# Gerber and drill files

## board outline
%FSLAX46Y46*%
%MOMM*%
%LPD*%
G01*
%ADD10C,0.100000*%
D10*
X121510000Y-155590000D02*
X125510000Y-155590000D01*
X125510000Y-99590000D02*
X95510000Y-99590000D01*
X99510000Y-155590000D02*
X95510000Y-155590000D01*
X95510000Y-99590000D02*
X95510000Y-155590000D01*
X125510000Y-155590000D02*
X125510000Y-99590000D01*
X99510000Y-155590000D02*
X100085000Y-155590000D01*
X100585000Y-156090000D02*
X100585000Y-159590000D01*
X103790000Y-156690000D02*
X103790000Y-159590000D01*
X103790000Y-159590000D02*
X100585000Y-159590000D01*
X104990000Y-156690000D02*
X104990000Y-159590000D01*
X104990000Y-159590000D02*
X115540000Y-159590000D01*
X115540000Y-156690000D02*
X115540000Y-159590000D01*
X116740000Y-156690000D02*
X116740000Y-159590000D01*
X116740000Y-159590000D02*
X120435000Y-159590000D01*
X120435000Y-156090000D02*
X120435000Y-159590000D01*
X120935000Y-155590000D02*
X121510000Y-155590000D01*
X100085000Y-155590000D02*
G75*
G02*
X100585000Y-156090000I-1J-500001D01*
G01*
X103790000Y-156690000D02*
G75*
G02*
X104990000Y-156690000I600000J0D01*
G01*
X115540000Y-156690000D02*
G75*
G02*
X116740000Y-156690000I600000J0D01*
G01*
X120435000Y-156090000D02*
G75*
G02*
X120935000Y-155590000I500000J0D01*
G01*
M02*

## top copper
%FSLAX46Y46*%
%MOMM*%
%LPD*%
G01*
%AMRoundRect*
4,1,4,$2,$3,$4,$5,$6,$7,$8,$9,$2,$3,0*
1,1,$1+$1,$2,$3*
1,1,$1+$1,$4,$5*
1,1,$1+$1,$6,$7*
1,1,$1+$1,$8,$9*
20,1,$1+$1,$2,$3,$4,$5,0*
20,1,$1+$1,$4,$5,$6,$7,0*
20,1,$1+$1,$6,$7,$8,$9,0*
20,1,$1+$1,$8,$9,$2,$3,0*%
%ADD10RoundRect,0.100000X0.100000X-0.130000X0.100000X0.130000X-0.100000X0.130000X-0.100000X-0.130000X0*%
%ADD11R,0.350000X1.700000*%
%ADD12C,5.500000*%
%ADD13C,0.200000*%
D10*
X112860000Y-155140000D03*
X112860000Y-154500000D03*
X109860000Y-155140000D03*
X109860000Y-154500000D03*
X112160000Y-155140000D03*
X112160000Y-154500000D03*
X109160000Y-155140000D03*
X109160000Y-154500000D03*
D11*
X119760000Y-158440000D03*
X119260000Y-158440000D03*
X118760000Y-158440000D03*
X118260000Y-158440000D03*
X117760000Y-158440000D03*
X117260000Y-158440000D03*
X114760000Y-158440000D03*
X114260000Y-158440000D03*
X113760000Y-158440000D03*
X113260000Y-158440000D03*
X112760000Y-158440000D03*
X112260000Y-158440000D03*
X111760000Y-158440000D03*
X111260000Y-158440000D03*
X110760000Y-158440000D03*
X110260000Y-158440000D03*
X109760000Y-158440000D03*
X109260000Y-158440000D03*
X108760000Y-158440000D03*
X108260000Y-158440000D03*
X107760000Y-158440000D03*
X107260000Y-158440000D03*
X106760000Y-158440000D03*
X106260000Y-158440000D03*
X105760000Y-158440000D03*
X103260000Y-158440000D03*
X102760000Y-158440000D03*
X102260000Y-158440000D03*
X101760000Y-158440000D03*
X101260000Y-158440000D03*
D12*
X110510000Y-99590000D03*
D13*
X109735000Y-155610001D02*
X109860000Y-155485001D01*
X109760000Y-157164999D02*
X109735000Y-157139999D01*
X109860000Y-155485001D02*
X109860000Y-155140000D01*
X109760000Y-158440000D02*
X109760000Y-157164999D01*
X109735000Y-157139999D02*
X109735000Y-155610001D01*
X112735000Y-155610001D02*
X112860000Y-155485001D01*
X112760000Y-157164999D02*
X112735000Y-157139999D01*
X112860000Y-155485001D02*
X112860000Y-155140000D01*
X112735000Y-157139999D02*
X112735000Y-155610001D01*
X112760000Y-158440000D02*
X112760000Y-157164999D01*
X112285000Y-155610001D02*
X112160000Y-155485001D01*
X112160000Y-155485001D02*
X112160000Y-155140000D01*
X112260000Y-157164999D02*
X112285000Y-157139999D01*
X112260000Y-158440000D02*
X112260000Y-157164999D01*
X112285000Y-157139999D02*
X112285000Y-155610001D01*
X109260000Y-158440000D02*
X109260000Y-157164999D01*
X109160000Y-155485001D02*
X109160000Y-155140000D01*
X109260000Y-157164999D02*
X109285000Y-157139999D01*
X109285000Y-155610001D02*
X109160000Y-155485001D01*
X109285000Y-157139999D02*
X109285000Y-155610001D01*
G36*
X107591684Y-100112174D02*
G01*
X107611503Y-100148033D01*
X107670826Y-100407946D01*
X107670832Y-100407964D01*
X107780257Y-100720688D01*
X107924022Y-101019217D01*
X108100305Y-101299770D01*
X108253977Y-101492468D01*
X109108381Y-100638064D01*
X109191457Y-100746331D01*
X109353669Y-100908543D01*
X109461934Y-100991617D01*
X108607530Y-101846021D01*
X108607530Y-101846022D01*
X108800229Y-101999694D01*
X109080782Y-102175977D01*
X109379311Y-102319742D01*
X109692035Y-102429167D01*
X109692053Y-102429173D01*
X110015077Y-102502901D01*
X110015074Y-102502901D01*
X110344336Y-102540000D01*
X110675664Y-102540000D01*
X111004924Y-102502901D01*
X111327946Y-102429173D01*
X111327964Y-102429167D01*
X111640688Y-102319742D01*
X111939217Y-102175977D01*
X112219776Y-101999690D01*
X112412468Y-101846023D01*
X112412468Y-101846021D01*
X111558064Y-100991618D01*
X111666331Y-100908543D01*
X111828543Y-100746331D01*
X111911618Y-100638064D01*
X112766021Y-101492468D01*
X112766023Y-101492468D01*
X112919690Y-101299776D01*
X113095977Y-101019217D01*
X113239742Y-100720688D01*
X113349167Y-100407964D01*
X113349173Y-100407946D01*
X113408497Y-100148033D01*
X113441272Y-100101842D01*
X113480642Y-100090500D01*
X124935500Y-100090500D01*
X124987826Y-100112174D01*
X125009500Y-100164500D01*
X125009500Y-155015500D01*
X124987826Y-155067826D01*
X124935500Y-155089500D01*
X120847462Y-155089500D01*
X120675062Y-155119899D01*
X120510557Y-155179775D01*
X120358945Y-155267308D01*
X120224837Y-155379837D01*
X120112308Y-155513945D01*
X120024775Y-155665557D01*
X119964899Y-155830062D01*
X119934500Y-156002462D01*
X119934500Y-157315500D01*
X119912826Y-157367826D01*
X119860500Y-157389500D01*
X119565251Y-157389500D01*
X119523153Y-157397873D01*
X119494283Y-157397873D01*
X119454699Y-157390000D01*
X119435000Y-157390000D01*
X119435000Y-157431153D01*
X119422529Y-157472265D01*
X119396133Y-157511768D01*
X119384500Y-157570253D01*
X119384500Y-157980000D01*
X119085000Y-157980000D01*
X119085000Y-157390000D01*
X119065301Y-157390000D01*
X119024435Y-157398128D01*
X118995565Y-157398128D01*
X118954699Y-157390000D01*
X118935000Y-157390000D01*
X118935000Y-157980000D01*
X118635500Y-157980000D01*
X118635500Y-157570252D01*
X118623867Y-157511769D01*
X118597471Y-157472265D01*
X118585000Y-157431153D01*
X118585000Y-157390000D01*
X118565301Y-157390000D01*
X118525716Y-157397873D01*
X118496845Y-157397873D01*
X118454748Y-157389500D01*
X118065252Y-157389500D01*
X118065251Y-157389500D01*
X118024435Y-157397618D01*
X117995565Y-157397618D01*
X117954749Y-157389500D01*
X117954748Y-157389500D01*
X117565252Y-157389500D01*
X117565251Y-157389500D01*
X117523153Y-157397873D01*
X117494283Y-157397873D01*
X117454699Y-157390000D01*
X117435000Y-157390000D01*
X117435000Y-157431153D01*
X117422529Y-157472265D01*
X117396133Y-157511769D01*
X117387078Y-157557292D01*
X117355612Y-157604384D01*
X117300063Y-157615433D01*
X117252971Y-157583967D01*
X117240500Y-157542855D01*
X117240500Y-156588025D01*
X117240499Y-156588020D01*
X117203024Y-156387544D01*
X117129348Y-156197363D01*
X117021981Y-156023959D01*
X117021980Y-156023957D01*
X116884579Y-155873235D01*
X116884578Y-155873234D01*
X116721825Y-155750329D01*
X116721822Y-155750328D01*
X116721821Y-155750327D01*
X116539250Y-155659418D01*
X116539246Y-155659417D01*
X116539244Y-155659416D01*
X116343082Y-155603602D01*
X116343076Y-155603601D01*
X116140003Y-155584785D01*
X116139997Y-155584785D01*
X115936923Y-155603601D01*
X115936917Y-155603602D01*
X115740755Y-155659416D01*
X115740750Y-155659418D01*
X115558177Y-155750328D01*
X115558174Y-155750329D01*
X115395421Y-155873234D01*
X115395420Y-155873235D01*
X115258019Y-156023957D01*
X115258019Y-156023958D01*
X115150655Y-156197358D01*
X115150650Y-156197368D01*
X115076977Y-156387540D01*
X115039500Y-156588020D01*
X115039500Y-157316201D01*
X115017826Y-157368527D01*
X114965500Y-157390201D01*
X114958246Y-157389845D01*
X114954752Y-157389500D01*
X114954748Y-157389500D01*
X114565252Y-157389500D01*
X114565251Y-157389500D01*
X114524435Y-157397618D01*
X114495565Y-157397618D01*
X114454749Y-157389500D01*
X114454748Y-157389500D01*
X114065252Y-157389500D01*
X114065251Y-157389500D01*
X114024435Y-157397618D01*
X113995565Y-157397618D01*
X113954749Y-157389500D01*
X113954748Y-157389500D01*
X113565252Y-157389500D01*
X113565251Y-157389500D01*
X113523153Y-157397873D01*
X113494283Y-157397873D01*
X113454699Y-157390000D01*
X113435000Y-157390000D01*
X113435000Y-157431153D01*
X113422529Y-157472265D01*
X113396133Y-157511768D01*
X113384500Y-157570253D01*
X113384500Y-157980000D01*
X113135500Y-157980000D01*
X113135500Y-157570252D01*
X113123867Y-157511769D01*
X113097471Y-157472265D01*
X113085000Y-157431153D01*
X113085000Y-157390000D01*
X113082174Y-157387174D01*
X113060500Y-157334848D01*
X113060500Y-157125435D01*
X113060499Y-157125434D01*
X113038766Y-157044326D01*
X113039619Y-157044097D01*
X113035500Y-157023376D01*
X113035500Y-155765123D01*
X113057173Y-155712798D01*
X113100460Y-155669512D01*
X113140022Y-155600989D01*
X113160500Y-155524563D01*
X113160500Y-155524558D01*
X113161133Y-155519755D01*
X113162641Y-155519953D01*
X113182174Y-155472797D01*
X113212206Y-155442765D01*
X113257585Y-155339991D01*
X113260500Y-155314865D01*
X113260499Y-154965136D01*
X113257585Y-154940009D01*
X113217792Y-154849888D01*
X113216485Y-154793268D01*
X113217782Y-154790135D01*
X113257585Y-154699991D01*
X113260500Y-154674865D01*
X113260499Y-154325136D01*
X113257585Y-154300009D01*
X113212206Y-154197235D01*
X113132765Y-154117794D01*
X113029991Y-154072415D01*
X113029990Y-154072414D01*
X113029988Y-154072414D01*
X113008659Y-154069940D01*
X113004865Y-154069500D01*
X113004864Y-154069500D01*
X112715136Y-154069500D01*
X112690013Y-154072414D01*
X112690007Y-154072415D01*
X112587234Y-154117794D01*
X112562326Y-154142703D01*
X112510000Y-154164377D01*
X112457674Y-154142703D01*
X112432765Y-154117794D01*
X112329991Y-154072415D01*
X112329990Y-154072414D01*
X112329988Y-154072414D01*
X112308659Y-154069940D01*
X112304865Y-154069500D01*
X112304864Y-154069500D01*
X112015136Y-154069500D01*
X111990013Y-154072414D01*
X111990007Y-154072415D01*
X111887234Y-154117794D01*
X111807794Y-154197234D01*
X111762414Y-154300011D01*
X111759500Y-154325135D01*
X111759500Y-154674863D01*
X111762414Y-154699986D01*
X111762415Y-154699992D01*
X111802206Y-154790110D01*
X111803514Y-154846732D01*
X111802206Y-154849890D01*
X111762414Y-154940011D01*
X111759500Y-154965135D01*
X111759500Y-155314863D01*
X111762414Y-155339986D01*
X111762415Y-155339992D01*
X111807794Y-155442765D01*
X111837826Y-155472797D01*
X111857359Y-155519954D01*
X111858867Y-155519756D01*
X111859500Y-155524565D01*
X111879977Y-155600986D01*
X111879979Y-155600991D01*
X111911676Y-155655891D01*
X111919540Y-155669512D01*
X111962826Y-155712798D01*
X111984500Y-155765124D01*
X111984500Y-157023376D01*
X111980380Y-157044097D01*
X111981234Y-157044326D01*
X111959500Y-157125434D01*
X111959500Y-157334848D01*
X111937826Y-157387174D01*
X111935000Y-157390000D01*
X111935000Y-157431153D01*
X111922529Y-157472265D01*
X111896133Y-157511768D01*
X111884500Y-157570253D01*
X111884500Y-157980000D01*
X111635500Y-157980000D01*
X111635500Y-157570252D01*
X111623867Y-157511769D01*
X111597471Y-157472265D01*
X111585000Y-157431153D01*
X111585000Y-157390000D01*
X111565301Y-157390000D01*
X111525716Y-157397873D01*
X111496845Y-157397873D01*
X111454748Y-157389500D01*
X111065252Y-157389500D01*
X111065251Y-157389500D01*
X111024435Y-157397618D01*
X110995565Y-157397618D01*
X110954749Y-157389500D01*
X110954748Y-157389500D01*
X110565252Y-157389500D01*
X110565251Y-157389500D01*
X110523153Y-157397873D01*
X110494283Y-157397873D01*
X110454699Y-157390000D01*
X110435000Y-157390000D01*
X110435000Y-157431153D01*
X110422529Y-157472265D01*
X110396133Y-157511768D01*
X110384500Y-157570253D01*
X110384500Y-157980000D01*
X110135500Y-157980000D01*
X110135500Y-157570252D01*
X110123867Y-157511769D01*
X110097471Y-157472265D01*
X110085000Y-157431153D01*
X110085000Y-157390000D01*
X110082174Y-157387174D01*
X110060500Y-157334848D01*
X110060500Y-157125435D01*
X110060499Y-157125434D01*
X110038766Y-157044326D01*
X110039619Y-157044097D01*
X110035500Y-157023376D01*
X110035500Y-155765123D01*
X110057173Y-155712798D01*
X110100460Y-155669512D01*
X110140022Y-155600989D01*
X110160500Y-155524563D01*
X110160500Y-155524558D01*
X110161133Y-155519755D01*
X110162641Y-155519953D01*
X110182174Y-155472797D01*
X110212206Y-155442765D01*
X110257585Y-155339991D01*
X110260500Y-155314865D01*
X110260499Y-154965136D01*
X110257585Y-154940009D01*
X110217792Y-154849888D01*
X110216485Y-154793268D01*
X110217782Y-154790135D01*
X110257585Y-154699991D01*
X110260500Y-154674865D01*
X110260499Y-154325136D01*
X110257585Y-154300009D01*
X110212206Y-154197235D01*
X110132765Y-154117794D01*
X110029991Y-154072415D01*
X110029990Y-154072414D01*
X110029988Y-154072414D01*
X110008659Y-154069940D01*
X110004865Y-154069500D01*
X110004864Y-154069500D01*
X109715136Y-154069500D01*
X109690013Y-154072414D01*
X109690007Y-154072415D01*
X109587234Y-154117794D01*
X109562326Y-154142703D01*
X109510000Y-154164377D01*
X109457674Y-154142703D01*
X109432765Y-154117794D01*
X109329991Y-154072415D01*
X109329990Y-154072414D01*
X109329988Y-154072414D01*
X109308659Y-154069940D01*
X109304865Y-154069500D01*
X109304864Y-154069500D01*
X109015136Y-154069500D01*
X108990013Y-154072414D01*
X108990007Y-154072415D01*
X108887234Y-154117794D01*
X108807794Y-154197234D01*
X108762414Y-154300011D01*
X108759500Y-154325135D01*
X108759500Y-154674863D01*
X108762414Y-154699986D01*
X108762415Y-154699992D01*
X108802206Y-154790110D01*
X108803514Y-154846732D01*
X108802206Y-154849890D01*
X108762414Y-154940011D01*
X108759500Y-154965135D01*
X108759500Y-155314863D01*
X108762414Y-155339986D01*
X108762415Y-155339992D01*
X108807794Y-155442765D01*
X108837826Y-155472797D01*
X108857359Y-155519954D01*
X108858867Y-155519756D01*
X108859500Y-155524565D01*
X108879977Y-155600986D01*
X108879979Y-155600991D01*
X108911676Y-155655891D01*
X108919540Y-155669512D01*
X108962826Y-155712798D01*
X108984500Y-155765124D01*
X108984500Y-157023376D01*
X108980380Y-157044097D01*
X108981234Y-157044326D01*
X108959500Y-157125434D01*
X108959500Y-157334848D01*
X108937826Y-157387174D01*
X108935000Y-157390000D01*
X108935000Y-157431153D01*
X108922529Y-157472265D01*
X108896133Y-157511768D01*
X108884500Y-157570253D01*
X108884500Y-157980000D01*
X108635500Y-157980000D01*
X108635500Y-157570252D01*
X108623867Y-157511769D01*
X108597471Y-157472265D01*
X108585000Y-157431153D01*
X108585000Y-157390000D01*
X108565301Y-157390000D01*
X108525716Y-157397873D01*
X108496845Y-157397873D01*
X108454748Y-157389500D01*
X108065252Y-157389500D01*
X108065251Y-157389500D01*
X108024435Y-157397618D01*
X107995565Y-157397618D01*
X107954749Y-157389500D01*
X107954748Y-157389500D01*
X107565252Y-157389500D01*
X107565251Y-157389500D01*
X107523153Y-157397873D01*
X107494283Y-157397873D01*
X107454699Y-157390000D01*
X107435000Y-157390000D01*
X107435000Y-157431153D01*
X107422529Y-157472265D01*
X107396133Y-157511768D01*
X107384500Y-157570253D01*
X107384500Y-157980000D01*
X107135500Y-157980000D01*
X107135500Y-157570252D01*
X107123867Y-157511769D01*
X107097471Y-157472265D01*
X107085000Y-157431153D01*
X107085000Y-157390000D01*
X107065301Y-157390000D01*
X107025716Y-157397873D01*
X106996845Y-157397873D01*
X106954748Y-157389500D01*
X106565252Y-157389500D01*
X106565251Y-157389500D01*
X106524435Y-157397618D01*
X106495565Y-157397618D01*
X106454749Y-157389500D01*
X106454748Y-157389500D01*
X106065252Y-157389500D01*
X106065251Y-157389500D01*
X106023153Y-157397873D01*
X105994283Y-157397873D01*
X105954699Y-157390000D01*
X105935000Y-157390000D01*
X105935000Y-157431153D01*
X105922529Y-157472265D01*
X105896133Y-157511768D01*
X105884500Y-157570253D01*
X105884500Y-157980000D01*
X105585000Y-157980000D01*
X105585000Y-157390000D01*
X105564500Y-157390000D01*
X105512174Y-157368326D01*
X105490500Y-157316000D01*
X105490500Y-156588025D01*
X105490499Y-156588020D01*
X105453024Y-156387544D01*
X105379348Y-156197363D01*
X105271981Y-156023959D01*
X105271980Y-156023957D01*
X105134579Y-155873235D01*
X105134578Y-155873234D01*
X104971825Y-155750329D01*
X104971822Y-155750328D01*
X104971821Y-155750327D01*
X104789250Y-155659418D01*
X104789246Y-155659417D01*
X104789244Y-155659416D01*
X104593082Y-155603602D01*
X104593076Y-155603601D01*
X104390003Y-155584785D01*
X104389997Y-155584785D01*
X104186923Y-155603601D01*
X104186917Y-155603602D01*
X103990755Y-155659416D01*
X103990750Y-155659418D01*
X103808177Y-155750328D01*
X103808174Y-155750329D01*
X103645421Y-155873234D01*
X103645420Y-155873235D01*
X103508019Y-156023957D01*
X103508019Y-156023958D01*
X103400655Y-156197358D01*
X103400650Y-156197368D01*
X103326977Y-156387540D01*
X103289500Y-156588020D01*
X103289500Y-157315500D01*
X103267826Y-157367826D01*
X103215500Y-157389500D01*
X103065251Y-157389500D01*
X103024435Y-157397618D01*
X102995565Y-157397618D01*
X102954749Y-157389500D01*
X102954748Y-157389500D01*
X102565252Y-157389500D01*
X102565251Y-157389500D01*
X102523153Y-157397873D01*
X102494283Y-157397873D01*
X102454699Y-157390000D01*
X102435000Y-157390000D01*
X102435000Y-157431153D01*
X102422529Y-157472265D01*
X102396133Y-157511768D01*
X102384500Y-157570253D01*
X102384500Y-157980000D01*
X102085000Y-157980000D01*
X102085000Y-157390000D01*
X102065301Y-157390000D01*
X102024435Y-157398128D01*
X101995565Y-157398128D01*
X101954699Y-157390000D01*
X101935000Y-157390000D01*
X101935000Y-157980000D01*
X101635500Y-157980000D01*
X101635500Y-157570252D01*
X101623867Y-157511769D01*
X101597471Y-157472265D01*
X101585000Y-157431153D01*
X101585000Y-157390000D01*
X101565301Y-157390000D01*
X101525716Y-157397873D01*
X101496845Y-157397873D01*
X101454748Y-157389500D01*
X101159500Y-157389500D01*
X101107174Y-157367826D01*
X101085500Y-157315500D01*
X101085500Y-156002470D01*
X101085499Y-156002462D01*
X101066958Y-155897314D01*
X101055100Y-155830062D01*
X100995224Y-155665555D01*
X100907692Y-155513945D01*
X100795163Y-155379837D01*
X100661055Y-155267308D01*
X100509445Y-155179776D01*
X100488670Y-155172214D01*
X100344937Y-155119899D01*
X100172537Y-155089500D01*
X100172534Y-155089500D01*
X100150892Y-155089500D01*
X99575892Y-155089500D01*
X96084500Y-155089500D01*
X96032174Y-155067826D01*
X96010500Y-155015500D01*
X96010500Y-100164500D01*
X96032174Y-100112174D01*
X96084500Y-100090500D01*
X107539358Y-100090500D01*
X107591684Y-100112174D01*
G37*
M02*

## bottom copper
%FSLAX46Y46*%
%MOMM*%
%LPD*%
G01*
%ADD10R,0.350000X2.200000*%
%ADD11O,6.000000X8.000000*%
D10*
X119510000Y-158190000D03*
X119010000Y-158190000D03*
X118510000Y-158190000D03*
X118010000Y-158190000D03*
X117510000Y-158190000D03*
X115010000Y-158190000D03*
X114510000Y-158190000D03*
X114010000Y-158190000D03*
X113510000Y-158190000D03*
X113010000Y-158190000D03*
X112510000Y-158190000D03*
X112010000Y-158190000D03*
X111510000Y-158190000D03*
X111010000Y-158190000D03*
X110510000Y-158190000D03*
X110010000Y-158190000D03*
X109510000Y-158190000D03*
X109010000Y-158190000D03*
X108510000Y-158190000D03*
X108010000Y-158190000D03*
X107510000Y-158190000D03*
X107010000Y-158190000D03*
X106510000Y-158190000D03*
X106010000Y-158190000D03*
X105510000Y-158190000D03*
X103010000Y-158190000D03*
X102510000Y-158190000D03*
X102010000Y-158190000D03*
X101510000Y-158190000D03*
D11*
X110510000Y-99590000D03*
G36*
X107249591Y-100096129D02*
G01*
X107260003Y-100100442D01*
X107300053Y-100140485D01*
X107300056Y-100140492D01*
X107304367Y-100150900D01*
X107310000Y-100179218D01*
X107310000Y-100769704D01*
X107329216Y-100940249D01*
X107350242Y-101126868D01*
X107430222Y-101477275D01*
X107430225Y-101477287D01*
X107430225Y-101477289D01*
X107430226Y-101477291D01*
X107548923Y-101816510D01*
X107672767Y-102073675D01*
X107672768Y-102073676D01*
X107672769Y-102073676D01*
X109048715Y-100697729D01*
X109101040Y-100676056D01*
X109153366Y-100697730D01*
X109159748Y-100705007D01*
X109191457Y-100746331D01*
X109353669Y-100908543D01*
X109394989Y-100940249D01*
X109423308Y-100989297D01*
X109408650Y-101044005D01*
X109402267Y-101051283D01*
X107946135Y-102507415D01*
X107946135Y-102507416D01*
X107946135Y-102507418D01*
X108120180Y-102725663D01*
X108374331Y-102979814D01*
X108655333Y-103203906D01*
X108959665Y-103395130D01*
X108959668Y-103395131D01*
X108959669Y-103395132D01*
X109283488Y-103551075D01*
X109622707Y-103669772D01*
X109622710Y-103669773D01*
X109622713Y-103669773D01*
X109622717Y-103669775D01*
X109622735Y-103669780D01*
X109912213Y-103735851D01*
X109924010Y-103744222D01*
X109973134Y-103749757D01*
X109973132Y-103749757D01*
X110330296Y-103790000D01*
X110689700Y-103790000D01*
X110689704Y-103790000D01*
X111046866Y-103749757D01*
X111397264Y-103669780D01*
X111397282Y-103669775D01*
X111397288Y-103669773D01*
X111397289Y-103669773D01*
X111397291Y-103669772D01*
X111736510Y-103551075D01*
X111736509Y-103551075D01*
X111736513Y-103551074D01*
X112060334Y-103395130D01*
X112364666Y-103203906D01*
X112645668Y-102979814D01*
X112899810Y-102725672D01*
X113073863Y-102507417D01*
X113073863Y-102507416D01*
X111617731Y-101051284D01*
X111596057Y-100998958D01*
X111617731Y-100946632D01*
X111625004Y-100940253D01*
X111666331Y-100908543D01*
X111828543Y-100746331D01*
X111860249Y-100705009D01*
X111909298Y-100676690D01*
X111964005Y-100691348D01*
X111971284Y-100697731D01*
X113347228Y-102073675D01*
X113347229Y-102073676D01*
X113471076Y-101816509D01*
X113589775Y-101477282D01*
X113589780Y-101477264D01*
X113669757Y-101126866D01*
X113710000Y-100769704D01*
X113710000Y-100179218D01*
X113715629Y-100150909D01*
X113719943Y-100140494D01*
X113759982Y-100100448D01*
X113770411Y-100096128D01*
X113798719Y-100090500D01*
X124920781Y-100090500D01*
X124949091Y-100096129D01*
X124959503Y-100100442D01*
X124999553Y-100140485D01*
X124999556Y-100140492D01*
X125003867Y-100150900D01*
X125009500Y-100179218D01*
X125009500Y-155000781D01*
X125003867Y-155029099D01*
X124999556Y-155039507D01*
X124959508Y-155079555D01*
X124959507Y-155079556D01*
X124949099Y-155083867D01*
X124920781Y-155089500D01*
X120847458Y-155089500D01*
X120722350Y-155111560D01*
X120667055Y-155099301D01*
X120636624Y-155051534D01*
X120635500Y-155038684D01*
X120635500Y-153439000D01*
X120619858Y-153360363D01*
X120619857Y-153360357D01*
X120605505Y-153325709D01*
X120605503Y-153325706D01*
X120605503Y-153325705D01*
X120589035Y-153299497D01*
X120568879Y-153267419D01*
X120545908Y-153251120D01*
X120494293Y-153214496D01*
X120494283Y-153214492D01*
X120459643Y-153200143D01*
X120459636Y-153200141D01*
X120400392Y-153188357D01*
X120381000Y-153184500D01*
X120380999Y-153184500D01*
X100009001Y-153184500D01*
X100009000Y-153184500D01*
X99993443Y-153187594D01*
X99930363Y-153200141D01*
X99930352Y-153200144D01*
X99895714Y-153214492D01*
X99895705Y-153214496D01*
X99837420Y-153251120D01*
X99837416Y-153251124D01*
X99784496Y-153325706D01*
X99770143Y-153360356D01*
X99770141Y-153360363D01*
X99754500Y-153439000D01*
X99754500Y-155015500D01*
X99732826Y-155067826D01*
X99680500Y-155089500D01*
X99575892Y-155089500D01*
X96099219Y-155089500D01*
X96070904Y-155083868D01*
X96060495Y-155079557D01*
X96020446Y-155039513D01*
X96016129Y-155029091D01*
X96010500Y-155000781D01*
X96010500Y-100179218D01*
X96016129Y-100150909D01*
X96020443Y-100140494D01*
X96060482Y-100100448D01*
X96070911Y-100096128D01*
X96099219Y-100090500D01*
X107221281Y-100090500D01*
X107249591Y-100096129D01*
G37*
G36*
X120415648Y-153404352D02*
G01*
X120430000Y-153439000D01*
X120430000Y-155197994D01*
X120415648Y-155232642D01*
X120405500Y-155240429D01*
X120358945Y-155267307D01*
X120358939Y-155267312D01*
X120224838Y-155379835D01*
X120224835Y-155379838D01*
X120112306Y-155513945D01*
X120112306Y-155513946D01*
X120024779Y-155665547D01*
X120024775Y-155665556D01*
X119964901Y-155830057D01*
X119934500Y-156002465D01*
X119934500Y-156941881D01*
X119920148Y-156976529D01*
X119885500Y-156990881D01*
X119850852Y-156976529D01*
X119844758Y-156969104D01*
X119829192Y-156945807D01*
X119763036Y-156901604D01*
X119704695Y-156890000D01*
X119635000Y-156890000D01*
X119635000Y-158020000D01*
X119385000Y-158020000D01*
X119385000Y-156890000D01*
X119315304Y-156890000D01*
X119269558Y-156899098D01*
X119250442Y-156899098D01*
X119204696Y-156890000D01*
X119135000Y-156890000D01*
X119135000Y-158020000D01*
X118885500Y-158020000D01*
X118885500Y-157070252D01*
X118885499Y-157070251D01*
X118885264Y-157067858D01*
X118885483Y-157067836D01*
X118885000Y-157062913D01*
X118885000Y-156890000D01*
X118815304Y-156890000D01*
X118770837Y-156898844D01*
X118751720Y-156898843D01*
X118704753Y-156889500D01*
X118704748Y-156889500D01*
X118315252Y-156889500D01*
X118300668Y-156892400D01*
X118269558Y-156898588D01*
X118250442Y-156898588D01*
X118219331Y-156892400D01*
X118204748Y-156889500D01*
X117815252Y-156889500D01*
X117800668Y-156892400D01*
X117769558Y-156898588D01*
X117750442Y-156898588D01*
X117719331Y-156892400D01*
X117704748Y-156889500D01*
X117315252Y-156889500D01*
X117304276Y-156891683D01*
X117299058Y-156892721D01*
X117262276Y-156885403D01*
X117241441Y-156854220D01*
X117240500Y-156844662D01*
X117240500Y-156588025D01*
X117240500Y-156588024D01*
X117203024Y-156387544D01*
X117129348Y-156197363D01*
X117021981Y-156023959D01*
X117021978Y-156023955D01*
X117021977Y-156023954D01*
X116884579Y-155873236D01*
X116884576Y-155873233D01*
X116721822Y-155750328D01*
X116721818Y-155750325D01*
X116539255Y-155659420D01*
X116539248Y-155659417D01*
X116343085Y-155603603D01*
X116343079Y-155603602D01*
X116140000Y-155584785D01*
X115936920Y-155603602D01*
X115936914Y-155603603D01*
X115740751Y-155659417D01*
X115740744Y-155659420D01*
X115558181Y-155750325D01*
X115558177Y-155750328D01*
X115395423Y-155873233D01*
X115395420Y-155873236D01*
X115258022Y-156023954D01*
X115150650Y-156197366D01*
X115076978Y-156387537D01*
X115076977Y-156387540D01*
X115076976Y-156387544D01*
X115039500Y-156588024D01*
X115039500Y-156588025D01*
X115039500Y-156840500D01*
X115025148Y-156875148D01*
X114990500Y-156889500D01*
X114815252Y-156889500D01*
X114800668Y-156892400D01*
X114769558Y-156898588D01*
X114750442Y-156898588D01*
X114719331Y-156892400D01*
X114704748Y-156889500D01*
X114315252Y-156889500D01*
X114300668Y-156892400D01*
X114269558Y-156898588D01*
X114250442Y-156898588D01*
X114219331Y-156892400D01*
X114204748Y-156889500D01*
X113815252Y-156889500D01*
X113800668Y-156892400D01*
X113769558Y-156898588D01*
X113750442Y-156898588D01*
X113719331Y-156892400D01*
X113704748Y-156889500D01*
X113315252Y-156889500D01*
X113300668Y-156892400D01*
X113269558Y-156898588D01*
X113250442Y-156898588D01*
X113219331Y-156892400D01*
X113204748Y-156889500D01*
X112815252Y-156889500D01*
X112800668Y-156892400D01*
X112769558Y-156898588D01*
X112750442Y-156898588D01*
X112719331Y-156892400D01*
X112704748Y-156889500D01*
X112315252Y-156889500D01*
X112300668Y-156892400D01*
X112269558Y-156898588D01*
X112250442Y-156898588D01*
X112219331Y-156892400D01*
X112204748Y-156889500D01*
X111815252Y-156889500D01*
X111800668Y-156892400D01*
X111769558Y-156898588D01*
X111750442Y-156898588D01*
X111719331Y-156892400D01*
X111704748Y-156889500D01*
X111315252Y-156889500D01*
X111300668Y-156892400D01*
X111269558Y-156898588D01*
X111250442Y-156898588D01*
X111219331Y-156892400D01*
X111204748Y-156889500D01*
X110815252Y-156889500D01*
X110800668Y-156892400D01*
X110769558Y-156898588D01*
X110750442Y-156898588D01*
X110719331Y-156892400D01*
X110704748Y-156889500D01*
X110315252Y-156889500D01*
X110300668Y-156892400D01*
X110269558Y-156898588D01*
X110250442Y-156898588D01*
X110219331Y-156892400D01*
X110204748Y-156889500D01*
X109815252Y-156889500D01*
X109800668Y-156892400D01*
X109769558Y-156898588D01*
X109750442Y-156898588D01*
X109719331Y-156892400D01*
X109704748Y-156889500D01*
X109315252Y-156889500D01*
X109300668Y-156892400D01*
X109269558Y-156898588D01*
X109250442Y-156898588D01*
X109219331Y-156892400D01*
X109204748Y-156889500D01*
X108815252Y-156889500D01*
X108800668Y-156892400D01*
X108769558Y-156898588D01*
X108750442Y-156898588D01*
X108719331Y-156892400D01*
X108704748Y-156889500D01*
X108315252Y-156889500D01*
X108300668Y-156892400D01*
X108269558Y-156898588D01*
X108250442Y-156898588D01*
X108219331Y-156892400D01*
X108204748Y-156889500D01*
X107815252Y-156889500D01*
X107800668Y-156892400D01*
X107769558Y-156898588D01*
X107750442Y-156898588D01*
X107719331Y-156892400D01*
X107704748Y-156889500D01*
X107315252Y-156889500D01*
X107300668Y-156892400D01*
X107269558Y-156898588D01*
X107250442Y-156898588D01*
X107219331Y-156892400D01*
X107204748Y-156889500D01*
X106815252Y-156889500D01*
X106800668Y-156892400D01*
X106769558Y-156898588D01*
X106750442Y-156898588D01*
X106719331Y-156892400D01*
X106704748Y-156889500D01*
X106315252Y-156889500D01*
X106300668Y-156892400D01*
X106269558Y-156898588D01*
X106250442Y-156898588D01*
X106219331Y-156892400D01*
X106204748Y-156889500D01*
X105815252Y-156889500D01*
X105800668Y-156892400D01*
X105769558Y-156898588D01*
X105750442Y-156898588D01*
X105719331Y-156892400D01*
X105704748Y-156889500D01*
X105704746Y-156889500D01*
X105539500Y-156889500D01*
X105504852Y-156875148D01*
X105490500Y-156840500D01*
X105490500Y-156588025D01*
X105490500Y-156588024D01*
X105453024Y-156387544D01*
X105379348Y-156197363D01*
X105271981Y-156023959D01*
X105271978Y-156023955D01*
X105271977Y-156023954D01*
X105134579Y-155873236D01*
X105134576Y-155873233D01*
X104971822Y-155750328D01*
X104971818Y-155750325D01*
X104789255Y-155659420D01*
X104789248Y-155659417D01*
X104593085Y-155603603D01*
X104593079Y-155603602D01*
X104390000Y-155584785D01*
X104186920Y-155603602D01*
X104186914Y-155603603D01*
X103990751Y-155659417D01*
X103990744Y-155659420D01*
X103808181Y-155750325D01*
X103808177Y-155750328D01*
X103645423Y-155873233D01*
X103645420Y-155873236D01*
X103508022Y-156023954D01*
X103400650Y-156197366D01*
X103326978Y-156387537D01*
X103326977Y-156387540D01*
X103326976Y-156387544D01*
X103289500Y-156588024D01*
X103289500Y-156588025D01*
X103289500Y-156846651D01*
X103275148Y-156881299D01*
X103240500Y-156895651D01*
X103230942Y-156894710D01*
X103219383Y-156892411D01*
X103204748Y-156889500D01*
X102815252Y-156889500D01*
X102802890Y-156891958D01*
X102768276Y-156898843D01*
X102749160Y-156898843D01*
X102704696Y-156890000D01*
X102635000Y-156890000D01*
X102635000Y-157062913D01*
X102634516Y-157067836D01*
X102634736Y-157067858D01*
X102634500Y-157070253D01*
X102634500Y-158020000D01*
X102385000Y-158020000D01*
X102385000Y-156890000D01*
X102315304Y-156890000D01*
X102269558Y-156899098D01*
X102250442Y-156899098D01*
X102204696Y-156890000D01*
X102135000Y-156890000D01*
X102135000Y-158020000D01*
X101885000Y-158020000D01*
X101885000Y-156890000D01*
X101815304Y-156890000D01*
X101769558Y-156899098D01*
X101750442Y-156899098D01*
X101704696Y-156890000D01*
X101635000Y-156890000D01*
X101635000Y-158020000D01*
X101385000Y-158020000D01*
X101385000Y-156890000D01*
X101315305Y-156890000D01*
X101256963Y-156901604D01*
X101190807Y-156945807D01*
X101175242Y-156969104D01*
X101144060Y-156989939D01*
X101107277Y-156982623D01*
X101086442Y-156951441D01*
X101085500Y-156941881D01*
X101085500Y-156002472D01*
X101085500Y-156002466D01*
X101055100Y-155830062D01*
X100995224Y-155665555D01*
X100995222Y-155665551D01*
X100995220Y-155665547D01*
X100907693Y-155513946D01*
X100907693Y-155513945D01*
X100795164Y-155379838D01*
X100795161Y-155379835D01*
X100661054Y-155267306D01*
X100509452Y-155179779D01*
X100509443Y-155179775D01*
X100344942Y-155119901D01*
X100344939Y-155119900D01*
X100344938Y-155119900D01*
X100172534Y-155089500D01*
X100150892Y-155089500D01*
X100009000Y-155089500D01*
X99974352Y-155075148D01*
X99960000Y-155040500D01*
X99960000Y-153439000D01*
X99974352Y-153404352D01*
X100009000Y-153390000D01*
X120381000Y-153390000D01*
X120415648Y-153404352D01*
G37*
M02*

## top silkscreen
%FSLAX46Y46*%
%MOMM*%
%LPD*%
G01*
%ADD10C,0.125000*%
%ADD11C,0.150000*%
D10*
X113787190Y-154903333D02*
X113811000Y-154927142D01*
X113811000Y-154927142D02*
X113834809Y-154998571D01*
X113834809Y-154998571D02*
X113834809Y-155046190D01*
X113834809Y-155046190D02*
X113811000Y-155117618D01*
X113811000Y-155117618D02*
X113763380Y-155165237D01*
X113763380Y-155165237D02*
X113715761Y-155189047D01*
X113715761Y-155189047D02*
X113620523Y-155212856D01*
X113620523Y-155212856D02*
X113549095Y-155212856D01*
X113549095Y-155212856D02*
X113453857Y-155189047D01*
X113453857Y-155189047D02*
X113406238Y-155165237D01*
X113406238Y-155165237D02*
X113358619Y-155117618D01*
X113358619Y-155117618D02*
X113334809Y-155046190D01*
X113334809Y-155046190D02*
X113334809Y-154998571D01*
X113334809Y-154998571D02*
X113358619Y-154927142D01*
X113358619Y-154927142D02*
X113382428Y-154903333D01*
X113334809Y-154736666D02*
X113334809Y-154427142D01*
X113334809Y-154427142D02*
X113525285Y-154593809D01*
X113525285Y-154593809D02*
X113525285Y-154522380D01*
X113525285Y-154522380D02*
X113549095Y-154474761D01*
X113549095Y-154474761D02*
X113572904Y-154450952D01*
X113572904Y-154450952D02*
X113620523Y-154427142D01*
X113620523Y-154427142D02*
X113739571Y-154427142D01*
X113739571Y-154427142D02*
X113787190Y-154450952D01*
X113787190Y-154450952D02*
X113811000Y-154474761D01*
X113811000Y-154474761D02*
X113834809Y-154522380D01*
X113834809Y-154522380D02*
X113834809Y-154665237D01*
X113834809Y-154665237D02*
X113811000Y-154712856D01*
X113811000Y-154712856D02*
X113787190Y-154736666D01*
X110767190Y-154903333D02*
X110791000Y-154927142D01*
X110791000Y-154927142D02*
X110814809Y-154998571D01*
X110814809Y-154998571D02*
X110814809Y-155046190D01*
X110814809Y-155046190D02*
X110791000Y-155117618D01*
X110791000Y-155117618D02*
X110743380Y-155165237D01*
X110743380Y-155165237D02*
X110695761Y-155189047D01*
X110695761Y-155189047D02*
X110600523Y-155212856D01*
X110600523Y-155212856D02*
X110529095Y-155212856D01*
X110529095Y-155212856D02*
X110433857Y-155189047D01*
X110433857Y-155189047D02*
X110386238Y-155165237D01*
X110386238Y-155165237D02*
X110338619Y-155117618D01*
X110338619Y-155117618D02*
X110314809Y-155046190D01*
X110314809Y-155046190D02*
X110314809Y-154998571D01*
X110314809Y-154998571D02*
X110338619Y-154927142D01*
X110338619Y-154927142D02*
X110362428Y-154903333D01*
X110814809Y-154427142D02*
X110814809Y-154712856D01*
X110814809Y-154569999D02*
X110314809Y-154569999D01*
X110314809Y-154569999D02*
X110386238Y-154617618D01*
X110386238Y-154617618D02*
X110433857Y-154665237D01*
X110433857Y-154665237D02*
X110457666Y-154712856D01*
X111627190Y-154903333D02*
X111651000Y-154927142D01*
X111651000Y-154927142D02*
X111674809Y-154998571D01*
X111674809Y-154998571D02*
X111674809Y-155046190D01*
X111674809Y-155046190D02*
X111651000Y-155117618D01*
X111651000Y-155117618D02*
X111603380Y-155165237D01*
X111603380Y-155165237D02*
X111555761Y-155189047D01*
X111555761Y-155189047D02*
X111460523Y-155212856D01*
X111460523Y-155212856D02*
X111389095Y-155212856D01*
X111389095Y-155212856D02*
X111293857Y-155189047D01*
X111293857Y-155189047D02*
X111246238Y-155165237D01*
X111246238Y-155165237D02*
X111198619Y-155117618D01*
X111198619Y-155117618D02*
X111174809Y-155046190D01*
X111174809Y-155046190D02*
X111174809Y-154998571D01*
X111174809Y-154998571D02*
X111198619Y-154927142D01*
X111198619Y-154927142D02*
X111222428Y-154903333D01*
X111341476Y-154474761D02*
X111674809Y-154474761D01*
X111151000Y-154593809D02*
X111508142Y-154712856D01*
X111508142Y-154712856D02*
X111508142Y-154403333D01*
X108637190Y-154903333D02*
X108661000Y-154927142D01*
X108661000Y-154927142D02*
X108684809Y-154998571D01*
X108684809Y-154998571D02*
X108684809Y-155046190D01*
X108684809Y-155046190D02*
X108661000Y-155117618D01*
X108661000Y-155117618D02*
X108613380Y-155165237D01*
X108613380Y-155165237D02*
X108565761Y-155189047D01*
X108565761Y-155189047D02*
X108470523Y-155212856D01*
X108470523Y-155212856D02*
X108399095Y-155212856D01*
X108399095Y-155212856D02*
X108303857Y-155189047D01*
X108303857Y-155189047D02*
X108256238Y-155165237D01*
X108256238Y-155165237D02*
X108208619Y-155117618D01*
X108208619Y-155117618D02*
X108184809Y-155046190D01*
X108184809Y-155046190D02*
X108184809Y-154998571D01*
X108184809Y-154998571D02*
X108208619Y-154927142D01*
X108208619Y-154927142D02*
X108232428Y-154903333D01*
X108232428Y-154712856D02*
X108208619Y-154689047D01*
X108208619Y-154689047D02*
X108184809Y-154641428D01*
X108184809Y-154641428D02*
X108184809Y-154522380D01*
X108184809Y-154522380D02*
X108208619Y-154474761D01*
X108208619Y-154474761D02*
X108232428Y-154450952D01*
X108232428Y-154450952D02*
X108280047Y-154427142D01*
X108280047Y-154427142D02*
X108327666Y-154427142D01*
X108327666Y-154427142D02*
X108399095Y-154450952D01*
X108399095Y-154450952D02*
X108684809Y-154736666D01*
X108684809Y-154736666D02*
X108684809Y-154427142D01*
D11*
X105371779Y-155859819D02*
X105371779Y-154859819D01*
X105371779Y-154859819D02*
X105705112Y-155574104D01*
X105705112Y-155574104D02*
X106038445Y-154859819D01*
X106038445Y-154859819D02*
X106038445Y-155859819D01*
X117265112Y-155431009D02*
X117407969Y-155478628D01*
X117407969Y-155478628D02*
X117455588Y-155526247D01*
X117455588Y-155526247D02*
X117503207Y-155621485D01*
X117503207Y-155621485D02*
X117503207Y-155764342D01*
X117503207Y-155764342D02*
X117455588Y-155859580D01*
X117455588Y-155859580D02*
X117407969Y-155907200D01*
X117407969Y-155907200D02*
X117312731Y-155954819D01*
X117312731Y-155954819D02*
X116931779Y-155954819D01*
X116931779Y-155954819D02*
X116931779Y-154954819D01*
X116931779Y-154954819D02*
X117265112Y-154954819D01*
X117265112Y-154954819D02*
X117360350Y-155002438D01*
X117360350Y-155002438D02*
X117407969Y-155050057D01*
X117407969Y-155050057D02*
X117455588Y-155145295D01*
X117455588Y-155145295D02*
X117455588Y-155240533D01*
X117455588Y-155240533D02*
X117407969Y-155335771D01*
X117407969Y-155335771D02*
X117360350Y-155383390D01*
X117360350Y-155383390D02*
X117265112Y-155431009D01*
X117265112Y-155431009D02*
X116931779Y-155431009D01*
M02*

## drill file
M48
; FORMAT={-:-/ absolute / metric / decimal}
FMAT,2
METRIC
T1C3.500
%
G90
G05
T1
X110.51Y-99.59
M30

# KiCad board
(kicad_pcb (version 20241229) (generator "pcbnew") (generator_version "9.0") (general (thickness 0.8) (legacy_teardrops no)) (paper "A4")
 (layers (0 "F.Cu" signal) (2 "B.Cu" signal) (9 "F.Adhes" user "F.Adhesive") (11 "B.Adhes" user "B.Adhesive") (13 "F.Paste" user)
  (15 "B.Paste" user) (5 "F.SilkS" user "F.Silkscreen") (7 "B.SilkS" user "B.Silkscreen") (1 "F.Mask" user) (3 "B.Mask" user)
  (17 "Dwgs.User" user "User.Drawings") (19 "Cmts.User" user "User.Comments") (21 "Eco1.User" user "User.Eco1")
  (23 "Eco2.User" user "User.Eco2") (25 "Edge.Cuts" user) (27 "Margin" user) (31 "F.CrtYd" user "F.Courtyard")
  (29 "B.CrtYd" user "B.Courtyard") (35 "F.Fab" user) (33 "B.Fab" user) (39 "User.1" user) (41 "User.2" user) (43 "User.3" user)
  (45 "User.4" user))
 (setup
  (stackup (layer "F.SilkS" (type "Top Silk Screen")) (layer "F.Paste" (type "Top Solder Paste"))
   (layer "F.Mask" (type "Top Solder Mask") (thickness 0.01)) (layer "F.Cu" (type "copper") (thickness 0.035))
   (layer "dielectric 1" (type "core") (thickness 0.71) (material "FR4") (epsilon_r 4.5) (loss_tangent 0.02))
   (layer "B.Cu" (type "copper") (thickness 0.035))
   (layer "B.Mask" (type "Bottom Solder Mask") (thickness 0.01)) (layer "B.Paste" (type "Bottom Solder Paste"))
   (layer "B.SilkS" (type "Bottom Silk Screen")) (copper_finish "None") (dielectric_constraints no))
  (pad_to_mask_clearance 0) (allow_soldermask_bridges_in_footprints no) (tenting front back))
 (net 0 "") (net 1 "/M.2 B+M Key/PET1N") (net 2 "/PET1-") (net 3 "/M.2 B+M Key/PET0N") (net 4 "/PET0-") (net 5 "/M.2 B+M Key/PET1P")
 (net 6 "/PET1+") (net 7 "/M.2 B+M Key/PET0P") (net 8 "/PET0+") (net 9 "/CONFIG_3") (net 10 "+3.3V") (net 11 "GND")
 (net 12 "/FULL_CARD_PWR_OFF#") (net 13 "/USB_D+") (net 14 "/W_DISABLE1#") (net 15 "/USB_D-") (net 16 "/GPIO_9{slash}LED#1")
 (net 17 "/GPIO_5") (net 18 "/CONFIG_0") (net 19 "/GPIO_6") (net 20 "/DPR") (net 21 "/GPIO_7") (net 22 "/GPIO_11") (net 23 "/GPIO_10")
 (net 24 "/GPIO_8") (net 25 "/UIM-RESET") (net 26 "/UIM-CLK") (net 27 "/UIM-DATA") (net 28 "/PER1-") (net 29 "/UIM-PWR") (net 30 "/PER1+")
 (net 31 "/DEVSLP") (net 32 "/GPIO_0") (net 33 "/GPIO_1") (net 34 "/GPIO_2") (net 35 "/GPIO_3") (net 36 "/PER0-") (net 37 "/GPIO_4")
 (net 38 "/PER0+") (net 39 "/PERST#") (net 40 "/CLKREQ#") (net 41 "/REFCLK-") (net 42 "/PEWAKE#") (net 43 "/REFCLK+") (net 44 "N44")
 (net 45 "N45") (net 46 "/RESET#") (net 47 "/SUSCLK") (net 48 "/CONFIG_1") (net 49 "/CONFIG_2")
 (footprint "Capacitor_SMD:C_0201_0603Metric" (layer "F.Cu") (at 112.86 154.82 90)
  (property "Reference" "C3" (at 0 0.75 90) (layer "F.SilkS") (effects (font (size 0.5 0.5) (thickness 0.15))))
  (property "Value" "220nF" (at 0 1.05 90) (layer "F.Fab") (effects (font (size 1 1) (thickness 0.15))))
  (pad "" smd roundrect (at -0.345 0 90) (size 0.318 0.36) (layers "F.Paste") (roundrect_rratio 0.25))
  (pad "" smd roundrect (at 0.345 0 90) (size 0.318 0.36) (layers "F.Paste") (roundrect_rratio 0.25))
  (pad "1" smd roundrect (at -0.32 0 90) (size 0.46 0.4) (layers "F.Cu" "F.Mask") (roundrect_rratio 0.25) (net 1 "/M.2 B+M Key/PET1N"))
  (pad "2" smd roundrect (at 0.32 0 90) (size 0.46 0.4) (layers "F.Cu" "F.Mask") (roundrect_rratio 0.25) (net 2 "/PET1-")))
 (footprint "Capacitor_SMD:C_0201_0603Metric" (layer "F.Cu") (at 109.86 154.82 90)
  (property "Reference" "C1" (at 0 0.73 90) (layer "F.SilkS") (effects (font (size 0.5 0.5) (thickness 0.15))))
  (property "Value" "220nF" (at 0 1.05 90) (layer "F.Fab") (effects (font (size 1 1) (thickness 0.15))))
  (pad "" smd roundrect (at -0.345 0 90) (size 0.318 0.36) (layers "F.Paste") (roundrect_rratio 0.25))
  (pad "" smd roundrect (at 0.345 0 90) (size 0.318 0.36) (layers "F.Paste") (roundrect_rratio 0.25))
  (pad "1" smd roundrect (at -0.32 0 90) (size 0.46 0.4) (layers "F.Cu" "F.Mask") (roundrect_rratio 0.25) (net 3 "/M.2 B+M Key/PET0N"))
  (pad "2" smd roundrect (at 0.32 0 90) (size 0.46 0.4) (layers "F.Cu" "F.Mask") (roundrect_rratio 0.25) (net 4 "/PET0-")))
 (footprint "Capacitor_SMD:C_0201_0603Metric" (layer "F.Cu") (at 112.16 154.82 90)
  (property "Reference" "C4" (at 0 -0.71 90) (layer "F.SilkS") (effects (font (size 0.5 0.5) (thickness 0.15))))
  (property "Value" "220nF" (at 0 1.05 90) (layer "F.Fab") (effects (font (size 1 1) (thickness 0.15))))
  (pad "" smd roundrect (at -0.345 0 90) (size 0.318 0.36) (layers "F.Paste") (roundrect_rratio 0.25))
  (pad "" smd roundrect (at 0.345 0 90) (size 0.318 0.36) (layers "F.Paste") (roundrect_rratio 0.25))
  (pad "1" smd roundrect (at -0.32 0 90) (size 0.46 0.4) (layers "F.Cu" "F.Mask") (roundrect_rratio 0.25) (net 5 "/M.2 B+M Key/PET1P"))
  (pad "2" smd roundrect (at 0.32 0 90) (size 0.46 0.4) (layers "F.Cu" "F.Mask") (roundrect_rratio 0.25) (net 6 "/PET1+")))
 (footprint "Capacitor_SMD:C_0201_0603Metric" (layer "F.Cu") (at 109.16 154.82 90)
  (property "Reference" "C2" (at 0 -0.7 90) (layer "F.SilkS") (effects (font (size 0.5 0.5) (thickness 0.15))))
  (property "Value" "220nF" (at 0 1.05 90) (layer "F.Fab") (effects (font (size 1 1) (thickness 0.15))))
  (pad "" smd roundrect (at -0.345 0 90) (size 0.318 0.36) (layers "F.Paste") (roundrect_rratio 0.25))
  (pad "" smd roundrect (at 0.345 0 90) (size 0.318 0.36) (layers "F.Paste") (roundrect_rratio 0.25))
  (pad "1" smd roundrect (at -0.32 0 90) (size 0.46 0.4) (layers "F.Cu" "F.Mask") (roundrect_rratio 0.25) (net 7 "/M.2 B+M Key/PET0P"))
  (pad "2" smd roundrect (at 0.32 0 90) (size 0.46 0.4) (layers "F.Cu" "F.Mask") (roundrect_rratio 0.25) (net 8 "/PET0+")))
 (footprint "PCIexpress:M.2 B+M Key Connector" (layer "F.Cu") (at 110.51 158.48)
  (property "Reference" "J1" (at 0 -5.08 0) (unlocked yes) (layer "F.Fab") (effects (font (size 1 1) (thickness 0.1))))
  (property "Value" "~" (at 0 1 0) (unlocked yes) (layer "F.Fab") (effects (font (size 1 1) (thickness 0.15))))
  (fp_line (start -11 -2.89) (end -10.425 -2.89) (stroke (width 0.1) (type default)) (layer "Edge.Cuts"))
  (fp_line (start -9.925 -2.39) (end -9.925 1.11) (stroke (width 0.1) (type default)) (layer "Edge.Cuts"))
  (fp_line (start -6.72 -1.79) (end -6.72 1.11) (stroke (width 0.1) (type default)) (layer "Edge.Cuts"))
  (fp_line (start -6.72 1.11) (end -9.925 1.11) (stroke (width 0.1) (type default)) (layer "Edge.Cuts"))
  (fp_line (start -5.52 -1.79) (end -5.52 1.11) (stroke (width 0.1) (type default)) (layer "Edge.Cuts"))
  (fp_line (start -5.52 1.11) (end 5.03 1.11) (stroke (width 0.1) (type default)) (layer "Edge.Cuts"))
  (fp_line (start 5.03 -1.79) (end 5.03 1.11) (stroke (width 0.1) (type default)) (layer "Edge.Cuts"))
  (fp_line (start 6.23 -1.79) (end 6.23 1.11) (stroke (width 0.1) (type default)) (layer "Edge.Cuts"))
  (fp_line (start 6.23 1.11) (end 9.925 1.11) (stroke (width 0.1) (type default)) (layer "Edge.Cuts"))
  (fp_line (start 9.925 -2.39) (end 9.925 1.11) (stroke (width 0.1) (type default)) (layer "Edge.Cuts"))
  (fp_line (start 10.425 -2.89) (end 11 -2.89) (stroke (width 0.1) (type default)) (layer "Edge.Cuts"))
  (fp_arc (start -10.425 -2.89) (mid -10.071447 -2.743553) (end -9.925 -2.39) (stroke (width 0.1) (type default)) (layer "Edge.Cuts"))
  (fp_arc (start -6.72 -1.79) (mid -6.12 -2.39) (end -5.52 -1.79) (stroke (width 0.1) (type default)) (layer "Edge.Cuts"))
  (fp_arc (start 5.03 -1.79) (mid 5.63 -2.39) (end 6.23 -1.79) (stroke (width 0.1) (type default)) (layer "Edge.Cuts"))
  (fp_arc (start 9.925 -2.39) (mid 10.071447 -2.743553) (end 10.425 -2.89) (stroke (width 0.1) (type default)) (layer "Edge.Cuts"))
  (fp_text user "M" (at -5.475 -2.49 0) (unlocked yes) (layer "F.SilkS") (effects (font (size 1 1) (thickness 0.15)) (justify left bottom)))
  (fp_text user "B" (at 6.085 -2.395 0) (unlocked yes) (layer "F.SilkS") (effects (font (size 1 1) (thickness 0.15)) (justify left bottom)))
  (pad "1" smd rect (at 9.25 -0.04 180) (size 0.35 1.7) (layers "F.Cu") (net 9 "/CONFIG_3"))
  (pad "2" smd rect (at 9 -0.29 180) (size 0.35 2.2) (layers "B.Cu") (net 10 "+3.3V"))
  (pad "3" smd rect (at 8.75 -0.04 180) (size 0.35 1.7) (layers "F.Cu") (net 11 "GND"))
  (pad "4" smd rect (at 8.5 -0.29 180) (size 0.35 2.2) (layers "B.Cu") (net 10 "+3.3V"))
  (pad "5" smd rect (at 8.25 -0.04 180) (size 0.35 1.7) (layers "F.Cu") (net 11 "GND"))
  (pad "6" smd rect (at 8 -0.29 180) (size 0.35 2.2) (layers "B.Cu") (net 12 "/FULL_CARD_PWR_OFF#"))
  (pad "7" smd rect (at 7.75 -0.04 180) (size 0.35 1.7) (layers "F.Cu") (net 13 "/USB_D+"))
  (pad "8" smd rect (at 7.5 -0.29 180) (size 0.35 2.2) (layers "B.Cu") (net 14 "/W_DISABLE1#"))
  (pad "9" smd rect (at 7.25 -0.04 180) (size 0.35 1.7) (layers "F.Cu") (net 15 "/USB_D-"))
  (pad "10" smd rect (at 7 -0.29 180) (size 0.35 2.2) (layers "B.Cu") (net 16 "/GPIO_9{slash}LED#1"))
  (pad "11" smd rect (at 6.75 -0.04 180) (size 0.35 1.7) (layers "F.Cu") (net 11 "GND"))
  (pad "20" smd rect (at 4.5 -0.29 180) (size 0.35 2.2) (layers "B.Cu") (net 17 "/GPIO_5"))
  (pad "21" smd rect (at 4.25 -0.04 180) (size 0.35 1.7) (layers "F.Cu") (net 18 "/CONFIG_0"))
  (pad "22" smd rect (at 4 -0.29 180) (size 0.35 2.2) (layers "B.Cu") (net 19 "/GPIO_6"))
  (pad "23" smd rect (at 3.75 -0.04 180) (size 0.35 1.7) (layers "F.Cu") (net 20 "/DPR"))
  (pad "24" smd rect (at 3.5 -0.29 180) (size 0.35 2.2) (layers "B.Cu") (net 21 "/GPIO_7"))
  (pad "25" smd rect (at 3.25 -0.04 180) (size 0.35 1.7) (layers "F.Cu") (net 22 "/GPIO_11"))
  (pad "26" smd rect (at 3 -0.29 180) (size 0.35 2.2) (layers "B.Cu") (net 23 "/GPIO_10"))
  (pad "27" smd rect (at 2.75 -0.04 180) (size 0.35 1.7) (layers "F.Cu") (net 11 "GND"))
  (pad "28" smd rect (at 2.5 -0.29 180) (size 0.35 2.2) (layers "B.Cu") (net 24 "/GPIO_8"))
  (pad "29" smd rect (at 2.25 -0.04 180) (size 0.35 1.7) (layers "F.Cu") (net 1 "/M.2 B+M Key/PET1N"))
  (pad "30" smd rect (at 2 -0.29 180) (size 0.35 2.2) (layers "B.Cu") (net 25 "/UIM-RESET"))
  (pad "31" smd rect (at 1.75 -0.04 180) (size 0.35 1.7) (layers "F.Cu") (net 5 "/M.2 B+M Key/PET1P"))
  (pad "32" smd rect (at 1.5 -0.29 180) (size 0.35 2.2) (layers "B.Cu") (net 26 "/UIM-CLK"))
  (pad "33" smd rect (at 1.25 -0.04 180) (size 0.35 1.7) (layers "F.Cu") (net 11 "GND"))
  (pad "34" smd rect (at 1 -0.29 180) (size 0.35 2.2) (layers "B.Cu") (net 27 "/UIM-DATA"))
  (pad "35" smd rect (at 0.75 -0.04 180) (size 0.35 1.7) (layers "F.Cu") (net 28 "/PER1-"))
  (pad "36" smd rect (at 0.5 -0.29 180) (size 0.35 2.2) (layers "B.Cu") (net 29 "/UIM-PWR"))
  (pad "37" smd rect (at 0.25 -0.04 180) (size 0.35 1.7) (layers "F.Cu") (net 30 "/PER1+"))
  (pad "38" smd rect (at 0 -0.29 180) (size 0.35 2.2) (layers "B.Cu") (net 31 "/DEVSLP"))
  (pad "39" smd rect (at -0.25 -0.04 180) (size 0.35 1.7) (layers "F.Cu") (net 11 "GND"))
  (pad "40" smd rect (at -0.5 -0.29 180) (size 0.35 2.2) (layers "B.Cu") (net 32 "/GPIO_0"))
  (pad "41" smd rect (at -0.75 -0.04 180) (size 0.35 1.7) (layers "F.Cu") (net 3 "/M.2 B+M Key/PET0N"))
  (pad "42" smd rect (at -1 -0.29 180) (size 0.35 2.2) (layers "B.Cu") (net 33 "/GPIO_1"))
  (pad "43" smd rect (at -1.25 -0.04 180) (size 0.35 1.7) (layers "F.Cu") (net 7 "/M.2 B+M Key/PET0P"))
  (pad "44" smd rect (at -1.5 -0.29 180) (size 0.35 2.2) (layers "B.Cu") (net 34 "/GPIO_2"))
  (pad "45" smd rect (at -1.75 -0.04 180) (size 0.35 1.7) (layers "F.Cu") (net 11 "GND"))
  (pad "46" smd rect (at -2 -0.29 180) (size 0.35 2.2) (layers "B.Cu") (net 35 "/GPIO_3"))
  (pad "47" smd rect (at -2.25 -0.04 180) (size 0.35 1.7) (layers "F.Cu") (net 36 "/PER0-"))
  (pad "48" smd rect (at -2.5 -0.29 180) (size 0.35 2.2) (layers "B.Cu") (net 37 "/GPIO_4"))
  (pad "49" smd rect (at -2.75 -0.04 180) (size 0.35 1.7) (layers "F.Cu") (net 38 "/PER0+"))
  (pad "50" smd rect (at -3 -0.29 180) (size 0.35 2.2) (layers "B.Cu") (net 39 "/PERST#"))
  (pad "51" smd rect (at -3.25 -0.04 180) (size 0.35 1.7) (layers "F.Cu") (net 11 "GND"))
  (pad "52" smd rect (at -3.5 -0.29 180) (size 0.35 2.2) (layers "B.Cu") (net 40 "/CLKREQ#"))
  (pad "53" smd rect (at -3.75 -0.04 180) (size 0.35 1.7) (layers "F.Cu") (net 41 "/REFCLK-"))
  (pad "54" smd rect (at -4 -0.29 180) (size 0.35 2.2) (layers "B.Cu") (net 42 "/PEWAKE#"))
  (pad "55" smd rect (at -4.25 -0.04 180) (size 0.35 1.7) (layers "F.Cu") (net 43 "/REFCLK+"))
  (pad "56" smd rect (at -4.5 -0.29 180) (size 0.35 2.2) (layers "B.Cu") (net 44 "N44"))
  (pad "57" smd rect (at -4.75 -0.04 180) (size 0.35 1.7) (layers "F.Cu") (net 11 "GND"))
  (pad "58" smd rect (at -5 -0.29 180) (size 0.35 2.2) (layers "B.Cu") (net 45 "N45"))
  (pad "67" smd rect (at -7.25 -0.04 180) (size 0.35 1.7) (layers "F.Cu") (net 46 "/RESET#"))
  (pad "68" smd rect (at -7.5 -0.29 180) (size 0.35 2.2) (layers "B.Cu") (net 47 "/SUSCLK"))
  (pad "69" smd rect (at -7.75 -0.04 180) (size 0.35 1.7) (layers "F.Cu") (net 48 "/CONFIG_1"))
  (pad "70" smd rect (at -8 -0.29 180) (size 0.35 2.2) (layers "B.Cu") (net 10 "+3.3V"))
  (pad "71" smd rect (at -8.25 -0.04 180) (size 0.35 1.7) (layers "F.Cu") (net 11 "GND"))
  (pad "72" smd rect (at -8.5 -0.29 180) (size 0.35 2.2) (layers "B.Cu") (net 10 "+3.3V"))
  (pad "73" smd rect (at -8.75 -0.04 180) (size 0.35 1.7) (layers "F.Cu") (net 11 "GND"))
  (pad "74" smd rect (at -9 -0.29 180) (size 0.35 2.2) (layers "B.Cu") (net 10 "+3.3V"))
  (pad "75" smd rect (at -9.25 -0.04 180) (size 0.35 1.7) (layers "F.Cu") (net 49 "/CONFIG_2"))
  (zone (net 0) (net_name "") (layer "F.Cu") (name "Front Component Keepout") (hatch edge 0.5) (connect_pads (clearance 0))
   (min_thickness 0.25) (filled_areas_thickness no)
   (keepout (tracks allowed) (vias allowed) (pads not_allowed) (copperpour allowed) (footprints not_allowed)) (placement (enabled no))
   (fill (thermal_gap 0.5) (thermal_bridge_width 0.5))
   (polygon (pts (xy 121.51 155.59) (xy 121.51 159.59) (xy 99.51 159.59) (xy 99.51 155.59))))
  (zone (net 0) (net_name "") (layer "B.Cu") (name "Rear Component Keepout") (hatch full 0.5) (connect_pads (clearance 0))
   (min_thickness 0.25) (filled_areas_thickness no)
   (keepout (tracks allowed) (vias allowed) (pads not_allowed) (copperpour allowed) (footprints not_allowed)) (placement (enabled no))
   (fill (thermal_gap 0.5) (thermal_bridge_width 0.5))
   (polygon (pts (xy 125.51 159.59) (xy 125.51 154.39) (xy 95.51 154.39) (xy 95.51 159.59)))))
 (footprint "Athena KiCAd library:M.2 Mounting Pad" (layer "F.Cu") (at 110.51 99.59)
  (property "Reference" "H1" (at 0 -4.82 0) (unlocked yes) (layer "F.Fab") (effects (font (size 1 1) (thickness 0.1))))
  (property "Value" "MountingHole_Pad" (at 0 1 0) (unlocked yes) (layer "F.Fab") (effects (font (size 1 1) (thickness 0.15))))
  (pad "1" thru_hole circle (at 0 0) (size 5.5 5.5) (drill 3.5) (layers "*.Cu" "*.Mask") (remove_unused_layers no) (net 11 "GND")
   (padstack (mode front_inner_back)
    (layer "Inner" (shape circle) (size 5.5 5.5) (zone_connect -1))
    (layer "B.Cu" (shape oval) (size 6 8) (thermal_bridge_angle 45) (zone_connect -1)))))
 (gr_line (start 121.51 155.59) (end 125.51 155.59) (stroke (width 0.1) (type default)) (layer "Edge.Cuts"))
 (gr_line (start 125.51 99.59) (end 95.51 99.59) (stroke (width 0.1) (type default)) (layer "Edge.Cuts"))
 (gr_line (start 99.51 155.59) (end 95.51 155.59) (stroke (width 0.1) (type default)) (layer "Edge.Cuts"))
 (gr_line (start 95.51 99.59) (end 95.51 155.59) (stroke (width 0.1) (type default)) (layer "Edge.Cuts"))
 (gr_line (start 125.51 155.59) (end 125.51 99.59) (stroke (width 0.1) (type default)) (layer "Edge.Cuts"))
 (segment (start 109.735 155.610001) (end 109.86 155.485001) (width 0.2) (layer "F.Cu") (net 3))
 (segment (start 109.76 157.164999) (end 109.735 157.139999) (width 0.2) (layer "F.Cu") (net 3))
 (segment (start 109.86 155.485001) (end 109.86 155.14) (width 0.2) (layer "F.Cu") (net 3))
 (segment (start 109.76 158.44) (end 109.76 157.164999) (width 0.2) (layer "F.Cu") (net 3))
 (segment (start 109.735 157.139999) (end 109.735 155.610001) (width 0.2) (layer "F.Cu") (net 3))
 (segment (start 112.735 155.610001) (end 112.86 155.485001) (width 0.2) (layer "F.Cu") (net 1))
 (segment (start 112.76 157.164999) (end 112.735 157.139999) (width 0.2) (layer "F.Cu") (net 1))
 (segment (start 112.86 155.485001) (end 112.86 155.14) (width 0.2) (layer "F.Cu") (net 1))
 (segment (start 112.735 157.139999) (end 112.735 155.610001) (width 0.2) (layer "F.Cu") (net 1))
 (segment (start 112.76 158.44) (end 112.76 157.164999) (width 0.2) (layer "F.Cu") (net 1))
 (segment (start 112.285 155.610001) (end 112.16 155.485001) (width 0.2) (layer "F.Cu") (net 5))
 (segment (start 112.16 155.485001) (end 112.16 155.14) (width 0.2) (layer "F.Cu") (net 5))
 (segment (start 112.26 157.164999) (end 112.285 157.139999) (width 0.2) (layer "F.Cu") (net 5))
 (segment (start 112.26 158.44) (end 112.26 157.164999) (width 0.2) (layer "F.Cu") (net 5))
 (segment (start 112.285 157.139999) (end 112.285 155.610001) (width 0.2) (layer "F.Cu") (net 5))
 (segment (start 109.26 158.44) (end 109.26 157.164999) (width 0.2) (layer "F.Cu") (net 7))
 (segment (start 109.16 155.485001) (end 109.16 155.14) (width 0.2) (layer "F.Cu") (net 7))
 (segment (start 109.26 157.164999) (end 109.285 157.139999) (width 0.2) (layer "F.Cu") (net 7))
 (segment (start 109.285 155.610001) (end 109.16 155.485001) (width 0.2) (layer "F.Cu") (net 7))
 (segment (start 109.285 157.139999) (end 109.285 155.610001) (width 0.2) (layer "F.Cu") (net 7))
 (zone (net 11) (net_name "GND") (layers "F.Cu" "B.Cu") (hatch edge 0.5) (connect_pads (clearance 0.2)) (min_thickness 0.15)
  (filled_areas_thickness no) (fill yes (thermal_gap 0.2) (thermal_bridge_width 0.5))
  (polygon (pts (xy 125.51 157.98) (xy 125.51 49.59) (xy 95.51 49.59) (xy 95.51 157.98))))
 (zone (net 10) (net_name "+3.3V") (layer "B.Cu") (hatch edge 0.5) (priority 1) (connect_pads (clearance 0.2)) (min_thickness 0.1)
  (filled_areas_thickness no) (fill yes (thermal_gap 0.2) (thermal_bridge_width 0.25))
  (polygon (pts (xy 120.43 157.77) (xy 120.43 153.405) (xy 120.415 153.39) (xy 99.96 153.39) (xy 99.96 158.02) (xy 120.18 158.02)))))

